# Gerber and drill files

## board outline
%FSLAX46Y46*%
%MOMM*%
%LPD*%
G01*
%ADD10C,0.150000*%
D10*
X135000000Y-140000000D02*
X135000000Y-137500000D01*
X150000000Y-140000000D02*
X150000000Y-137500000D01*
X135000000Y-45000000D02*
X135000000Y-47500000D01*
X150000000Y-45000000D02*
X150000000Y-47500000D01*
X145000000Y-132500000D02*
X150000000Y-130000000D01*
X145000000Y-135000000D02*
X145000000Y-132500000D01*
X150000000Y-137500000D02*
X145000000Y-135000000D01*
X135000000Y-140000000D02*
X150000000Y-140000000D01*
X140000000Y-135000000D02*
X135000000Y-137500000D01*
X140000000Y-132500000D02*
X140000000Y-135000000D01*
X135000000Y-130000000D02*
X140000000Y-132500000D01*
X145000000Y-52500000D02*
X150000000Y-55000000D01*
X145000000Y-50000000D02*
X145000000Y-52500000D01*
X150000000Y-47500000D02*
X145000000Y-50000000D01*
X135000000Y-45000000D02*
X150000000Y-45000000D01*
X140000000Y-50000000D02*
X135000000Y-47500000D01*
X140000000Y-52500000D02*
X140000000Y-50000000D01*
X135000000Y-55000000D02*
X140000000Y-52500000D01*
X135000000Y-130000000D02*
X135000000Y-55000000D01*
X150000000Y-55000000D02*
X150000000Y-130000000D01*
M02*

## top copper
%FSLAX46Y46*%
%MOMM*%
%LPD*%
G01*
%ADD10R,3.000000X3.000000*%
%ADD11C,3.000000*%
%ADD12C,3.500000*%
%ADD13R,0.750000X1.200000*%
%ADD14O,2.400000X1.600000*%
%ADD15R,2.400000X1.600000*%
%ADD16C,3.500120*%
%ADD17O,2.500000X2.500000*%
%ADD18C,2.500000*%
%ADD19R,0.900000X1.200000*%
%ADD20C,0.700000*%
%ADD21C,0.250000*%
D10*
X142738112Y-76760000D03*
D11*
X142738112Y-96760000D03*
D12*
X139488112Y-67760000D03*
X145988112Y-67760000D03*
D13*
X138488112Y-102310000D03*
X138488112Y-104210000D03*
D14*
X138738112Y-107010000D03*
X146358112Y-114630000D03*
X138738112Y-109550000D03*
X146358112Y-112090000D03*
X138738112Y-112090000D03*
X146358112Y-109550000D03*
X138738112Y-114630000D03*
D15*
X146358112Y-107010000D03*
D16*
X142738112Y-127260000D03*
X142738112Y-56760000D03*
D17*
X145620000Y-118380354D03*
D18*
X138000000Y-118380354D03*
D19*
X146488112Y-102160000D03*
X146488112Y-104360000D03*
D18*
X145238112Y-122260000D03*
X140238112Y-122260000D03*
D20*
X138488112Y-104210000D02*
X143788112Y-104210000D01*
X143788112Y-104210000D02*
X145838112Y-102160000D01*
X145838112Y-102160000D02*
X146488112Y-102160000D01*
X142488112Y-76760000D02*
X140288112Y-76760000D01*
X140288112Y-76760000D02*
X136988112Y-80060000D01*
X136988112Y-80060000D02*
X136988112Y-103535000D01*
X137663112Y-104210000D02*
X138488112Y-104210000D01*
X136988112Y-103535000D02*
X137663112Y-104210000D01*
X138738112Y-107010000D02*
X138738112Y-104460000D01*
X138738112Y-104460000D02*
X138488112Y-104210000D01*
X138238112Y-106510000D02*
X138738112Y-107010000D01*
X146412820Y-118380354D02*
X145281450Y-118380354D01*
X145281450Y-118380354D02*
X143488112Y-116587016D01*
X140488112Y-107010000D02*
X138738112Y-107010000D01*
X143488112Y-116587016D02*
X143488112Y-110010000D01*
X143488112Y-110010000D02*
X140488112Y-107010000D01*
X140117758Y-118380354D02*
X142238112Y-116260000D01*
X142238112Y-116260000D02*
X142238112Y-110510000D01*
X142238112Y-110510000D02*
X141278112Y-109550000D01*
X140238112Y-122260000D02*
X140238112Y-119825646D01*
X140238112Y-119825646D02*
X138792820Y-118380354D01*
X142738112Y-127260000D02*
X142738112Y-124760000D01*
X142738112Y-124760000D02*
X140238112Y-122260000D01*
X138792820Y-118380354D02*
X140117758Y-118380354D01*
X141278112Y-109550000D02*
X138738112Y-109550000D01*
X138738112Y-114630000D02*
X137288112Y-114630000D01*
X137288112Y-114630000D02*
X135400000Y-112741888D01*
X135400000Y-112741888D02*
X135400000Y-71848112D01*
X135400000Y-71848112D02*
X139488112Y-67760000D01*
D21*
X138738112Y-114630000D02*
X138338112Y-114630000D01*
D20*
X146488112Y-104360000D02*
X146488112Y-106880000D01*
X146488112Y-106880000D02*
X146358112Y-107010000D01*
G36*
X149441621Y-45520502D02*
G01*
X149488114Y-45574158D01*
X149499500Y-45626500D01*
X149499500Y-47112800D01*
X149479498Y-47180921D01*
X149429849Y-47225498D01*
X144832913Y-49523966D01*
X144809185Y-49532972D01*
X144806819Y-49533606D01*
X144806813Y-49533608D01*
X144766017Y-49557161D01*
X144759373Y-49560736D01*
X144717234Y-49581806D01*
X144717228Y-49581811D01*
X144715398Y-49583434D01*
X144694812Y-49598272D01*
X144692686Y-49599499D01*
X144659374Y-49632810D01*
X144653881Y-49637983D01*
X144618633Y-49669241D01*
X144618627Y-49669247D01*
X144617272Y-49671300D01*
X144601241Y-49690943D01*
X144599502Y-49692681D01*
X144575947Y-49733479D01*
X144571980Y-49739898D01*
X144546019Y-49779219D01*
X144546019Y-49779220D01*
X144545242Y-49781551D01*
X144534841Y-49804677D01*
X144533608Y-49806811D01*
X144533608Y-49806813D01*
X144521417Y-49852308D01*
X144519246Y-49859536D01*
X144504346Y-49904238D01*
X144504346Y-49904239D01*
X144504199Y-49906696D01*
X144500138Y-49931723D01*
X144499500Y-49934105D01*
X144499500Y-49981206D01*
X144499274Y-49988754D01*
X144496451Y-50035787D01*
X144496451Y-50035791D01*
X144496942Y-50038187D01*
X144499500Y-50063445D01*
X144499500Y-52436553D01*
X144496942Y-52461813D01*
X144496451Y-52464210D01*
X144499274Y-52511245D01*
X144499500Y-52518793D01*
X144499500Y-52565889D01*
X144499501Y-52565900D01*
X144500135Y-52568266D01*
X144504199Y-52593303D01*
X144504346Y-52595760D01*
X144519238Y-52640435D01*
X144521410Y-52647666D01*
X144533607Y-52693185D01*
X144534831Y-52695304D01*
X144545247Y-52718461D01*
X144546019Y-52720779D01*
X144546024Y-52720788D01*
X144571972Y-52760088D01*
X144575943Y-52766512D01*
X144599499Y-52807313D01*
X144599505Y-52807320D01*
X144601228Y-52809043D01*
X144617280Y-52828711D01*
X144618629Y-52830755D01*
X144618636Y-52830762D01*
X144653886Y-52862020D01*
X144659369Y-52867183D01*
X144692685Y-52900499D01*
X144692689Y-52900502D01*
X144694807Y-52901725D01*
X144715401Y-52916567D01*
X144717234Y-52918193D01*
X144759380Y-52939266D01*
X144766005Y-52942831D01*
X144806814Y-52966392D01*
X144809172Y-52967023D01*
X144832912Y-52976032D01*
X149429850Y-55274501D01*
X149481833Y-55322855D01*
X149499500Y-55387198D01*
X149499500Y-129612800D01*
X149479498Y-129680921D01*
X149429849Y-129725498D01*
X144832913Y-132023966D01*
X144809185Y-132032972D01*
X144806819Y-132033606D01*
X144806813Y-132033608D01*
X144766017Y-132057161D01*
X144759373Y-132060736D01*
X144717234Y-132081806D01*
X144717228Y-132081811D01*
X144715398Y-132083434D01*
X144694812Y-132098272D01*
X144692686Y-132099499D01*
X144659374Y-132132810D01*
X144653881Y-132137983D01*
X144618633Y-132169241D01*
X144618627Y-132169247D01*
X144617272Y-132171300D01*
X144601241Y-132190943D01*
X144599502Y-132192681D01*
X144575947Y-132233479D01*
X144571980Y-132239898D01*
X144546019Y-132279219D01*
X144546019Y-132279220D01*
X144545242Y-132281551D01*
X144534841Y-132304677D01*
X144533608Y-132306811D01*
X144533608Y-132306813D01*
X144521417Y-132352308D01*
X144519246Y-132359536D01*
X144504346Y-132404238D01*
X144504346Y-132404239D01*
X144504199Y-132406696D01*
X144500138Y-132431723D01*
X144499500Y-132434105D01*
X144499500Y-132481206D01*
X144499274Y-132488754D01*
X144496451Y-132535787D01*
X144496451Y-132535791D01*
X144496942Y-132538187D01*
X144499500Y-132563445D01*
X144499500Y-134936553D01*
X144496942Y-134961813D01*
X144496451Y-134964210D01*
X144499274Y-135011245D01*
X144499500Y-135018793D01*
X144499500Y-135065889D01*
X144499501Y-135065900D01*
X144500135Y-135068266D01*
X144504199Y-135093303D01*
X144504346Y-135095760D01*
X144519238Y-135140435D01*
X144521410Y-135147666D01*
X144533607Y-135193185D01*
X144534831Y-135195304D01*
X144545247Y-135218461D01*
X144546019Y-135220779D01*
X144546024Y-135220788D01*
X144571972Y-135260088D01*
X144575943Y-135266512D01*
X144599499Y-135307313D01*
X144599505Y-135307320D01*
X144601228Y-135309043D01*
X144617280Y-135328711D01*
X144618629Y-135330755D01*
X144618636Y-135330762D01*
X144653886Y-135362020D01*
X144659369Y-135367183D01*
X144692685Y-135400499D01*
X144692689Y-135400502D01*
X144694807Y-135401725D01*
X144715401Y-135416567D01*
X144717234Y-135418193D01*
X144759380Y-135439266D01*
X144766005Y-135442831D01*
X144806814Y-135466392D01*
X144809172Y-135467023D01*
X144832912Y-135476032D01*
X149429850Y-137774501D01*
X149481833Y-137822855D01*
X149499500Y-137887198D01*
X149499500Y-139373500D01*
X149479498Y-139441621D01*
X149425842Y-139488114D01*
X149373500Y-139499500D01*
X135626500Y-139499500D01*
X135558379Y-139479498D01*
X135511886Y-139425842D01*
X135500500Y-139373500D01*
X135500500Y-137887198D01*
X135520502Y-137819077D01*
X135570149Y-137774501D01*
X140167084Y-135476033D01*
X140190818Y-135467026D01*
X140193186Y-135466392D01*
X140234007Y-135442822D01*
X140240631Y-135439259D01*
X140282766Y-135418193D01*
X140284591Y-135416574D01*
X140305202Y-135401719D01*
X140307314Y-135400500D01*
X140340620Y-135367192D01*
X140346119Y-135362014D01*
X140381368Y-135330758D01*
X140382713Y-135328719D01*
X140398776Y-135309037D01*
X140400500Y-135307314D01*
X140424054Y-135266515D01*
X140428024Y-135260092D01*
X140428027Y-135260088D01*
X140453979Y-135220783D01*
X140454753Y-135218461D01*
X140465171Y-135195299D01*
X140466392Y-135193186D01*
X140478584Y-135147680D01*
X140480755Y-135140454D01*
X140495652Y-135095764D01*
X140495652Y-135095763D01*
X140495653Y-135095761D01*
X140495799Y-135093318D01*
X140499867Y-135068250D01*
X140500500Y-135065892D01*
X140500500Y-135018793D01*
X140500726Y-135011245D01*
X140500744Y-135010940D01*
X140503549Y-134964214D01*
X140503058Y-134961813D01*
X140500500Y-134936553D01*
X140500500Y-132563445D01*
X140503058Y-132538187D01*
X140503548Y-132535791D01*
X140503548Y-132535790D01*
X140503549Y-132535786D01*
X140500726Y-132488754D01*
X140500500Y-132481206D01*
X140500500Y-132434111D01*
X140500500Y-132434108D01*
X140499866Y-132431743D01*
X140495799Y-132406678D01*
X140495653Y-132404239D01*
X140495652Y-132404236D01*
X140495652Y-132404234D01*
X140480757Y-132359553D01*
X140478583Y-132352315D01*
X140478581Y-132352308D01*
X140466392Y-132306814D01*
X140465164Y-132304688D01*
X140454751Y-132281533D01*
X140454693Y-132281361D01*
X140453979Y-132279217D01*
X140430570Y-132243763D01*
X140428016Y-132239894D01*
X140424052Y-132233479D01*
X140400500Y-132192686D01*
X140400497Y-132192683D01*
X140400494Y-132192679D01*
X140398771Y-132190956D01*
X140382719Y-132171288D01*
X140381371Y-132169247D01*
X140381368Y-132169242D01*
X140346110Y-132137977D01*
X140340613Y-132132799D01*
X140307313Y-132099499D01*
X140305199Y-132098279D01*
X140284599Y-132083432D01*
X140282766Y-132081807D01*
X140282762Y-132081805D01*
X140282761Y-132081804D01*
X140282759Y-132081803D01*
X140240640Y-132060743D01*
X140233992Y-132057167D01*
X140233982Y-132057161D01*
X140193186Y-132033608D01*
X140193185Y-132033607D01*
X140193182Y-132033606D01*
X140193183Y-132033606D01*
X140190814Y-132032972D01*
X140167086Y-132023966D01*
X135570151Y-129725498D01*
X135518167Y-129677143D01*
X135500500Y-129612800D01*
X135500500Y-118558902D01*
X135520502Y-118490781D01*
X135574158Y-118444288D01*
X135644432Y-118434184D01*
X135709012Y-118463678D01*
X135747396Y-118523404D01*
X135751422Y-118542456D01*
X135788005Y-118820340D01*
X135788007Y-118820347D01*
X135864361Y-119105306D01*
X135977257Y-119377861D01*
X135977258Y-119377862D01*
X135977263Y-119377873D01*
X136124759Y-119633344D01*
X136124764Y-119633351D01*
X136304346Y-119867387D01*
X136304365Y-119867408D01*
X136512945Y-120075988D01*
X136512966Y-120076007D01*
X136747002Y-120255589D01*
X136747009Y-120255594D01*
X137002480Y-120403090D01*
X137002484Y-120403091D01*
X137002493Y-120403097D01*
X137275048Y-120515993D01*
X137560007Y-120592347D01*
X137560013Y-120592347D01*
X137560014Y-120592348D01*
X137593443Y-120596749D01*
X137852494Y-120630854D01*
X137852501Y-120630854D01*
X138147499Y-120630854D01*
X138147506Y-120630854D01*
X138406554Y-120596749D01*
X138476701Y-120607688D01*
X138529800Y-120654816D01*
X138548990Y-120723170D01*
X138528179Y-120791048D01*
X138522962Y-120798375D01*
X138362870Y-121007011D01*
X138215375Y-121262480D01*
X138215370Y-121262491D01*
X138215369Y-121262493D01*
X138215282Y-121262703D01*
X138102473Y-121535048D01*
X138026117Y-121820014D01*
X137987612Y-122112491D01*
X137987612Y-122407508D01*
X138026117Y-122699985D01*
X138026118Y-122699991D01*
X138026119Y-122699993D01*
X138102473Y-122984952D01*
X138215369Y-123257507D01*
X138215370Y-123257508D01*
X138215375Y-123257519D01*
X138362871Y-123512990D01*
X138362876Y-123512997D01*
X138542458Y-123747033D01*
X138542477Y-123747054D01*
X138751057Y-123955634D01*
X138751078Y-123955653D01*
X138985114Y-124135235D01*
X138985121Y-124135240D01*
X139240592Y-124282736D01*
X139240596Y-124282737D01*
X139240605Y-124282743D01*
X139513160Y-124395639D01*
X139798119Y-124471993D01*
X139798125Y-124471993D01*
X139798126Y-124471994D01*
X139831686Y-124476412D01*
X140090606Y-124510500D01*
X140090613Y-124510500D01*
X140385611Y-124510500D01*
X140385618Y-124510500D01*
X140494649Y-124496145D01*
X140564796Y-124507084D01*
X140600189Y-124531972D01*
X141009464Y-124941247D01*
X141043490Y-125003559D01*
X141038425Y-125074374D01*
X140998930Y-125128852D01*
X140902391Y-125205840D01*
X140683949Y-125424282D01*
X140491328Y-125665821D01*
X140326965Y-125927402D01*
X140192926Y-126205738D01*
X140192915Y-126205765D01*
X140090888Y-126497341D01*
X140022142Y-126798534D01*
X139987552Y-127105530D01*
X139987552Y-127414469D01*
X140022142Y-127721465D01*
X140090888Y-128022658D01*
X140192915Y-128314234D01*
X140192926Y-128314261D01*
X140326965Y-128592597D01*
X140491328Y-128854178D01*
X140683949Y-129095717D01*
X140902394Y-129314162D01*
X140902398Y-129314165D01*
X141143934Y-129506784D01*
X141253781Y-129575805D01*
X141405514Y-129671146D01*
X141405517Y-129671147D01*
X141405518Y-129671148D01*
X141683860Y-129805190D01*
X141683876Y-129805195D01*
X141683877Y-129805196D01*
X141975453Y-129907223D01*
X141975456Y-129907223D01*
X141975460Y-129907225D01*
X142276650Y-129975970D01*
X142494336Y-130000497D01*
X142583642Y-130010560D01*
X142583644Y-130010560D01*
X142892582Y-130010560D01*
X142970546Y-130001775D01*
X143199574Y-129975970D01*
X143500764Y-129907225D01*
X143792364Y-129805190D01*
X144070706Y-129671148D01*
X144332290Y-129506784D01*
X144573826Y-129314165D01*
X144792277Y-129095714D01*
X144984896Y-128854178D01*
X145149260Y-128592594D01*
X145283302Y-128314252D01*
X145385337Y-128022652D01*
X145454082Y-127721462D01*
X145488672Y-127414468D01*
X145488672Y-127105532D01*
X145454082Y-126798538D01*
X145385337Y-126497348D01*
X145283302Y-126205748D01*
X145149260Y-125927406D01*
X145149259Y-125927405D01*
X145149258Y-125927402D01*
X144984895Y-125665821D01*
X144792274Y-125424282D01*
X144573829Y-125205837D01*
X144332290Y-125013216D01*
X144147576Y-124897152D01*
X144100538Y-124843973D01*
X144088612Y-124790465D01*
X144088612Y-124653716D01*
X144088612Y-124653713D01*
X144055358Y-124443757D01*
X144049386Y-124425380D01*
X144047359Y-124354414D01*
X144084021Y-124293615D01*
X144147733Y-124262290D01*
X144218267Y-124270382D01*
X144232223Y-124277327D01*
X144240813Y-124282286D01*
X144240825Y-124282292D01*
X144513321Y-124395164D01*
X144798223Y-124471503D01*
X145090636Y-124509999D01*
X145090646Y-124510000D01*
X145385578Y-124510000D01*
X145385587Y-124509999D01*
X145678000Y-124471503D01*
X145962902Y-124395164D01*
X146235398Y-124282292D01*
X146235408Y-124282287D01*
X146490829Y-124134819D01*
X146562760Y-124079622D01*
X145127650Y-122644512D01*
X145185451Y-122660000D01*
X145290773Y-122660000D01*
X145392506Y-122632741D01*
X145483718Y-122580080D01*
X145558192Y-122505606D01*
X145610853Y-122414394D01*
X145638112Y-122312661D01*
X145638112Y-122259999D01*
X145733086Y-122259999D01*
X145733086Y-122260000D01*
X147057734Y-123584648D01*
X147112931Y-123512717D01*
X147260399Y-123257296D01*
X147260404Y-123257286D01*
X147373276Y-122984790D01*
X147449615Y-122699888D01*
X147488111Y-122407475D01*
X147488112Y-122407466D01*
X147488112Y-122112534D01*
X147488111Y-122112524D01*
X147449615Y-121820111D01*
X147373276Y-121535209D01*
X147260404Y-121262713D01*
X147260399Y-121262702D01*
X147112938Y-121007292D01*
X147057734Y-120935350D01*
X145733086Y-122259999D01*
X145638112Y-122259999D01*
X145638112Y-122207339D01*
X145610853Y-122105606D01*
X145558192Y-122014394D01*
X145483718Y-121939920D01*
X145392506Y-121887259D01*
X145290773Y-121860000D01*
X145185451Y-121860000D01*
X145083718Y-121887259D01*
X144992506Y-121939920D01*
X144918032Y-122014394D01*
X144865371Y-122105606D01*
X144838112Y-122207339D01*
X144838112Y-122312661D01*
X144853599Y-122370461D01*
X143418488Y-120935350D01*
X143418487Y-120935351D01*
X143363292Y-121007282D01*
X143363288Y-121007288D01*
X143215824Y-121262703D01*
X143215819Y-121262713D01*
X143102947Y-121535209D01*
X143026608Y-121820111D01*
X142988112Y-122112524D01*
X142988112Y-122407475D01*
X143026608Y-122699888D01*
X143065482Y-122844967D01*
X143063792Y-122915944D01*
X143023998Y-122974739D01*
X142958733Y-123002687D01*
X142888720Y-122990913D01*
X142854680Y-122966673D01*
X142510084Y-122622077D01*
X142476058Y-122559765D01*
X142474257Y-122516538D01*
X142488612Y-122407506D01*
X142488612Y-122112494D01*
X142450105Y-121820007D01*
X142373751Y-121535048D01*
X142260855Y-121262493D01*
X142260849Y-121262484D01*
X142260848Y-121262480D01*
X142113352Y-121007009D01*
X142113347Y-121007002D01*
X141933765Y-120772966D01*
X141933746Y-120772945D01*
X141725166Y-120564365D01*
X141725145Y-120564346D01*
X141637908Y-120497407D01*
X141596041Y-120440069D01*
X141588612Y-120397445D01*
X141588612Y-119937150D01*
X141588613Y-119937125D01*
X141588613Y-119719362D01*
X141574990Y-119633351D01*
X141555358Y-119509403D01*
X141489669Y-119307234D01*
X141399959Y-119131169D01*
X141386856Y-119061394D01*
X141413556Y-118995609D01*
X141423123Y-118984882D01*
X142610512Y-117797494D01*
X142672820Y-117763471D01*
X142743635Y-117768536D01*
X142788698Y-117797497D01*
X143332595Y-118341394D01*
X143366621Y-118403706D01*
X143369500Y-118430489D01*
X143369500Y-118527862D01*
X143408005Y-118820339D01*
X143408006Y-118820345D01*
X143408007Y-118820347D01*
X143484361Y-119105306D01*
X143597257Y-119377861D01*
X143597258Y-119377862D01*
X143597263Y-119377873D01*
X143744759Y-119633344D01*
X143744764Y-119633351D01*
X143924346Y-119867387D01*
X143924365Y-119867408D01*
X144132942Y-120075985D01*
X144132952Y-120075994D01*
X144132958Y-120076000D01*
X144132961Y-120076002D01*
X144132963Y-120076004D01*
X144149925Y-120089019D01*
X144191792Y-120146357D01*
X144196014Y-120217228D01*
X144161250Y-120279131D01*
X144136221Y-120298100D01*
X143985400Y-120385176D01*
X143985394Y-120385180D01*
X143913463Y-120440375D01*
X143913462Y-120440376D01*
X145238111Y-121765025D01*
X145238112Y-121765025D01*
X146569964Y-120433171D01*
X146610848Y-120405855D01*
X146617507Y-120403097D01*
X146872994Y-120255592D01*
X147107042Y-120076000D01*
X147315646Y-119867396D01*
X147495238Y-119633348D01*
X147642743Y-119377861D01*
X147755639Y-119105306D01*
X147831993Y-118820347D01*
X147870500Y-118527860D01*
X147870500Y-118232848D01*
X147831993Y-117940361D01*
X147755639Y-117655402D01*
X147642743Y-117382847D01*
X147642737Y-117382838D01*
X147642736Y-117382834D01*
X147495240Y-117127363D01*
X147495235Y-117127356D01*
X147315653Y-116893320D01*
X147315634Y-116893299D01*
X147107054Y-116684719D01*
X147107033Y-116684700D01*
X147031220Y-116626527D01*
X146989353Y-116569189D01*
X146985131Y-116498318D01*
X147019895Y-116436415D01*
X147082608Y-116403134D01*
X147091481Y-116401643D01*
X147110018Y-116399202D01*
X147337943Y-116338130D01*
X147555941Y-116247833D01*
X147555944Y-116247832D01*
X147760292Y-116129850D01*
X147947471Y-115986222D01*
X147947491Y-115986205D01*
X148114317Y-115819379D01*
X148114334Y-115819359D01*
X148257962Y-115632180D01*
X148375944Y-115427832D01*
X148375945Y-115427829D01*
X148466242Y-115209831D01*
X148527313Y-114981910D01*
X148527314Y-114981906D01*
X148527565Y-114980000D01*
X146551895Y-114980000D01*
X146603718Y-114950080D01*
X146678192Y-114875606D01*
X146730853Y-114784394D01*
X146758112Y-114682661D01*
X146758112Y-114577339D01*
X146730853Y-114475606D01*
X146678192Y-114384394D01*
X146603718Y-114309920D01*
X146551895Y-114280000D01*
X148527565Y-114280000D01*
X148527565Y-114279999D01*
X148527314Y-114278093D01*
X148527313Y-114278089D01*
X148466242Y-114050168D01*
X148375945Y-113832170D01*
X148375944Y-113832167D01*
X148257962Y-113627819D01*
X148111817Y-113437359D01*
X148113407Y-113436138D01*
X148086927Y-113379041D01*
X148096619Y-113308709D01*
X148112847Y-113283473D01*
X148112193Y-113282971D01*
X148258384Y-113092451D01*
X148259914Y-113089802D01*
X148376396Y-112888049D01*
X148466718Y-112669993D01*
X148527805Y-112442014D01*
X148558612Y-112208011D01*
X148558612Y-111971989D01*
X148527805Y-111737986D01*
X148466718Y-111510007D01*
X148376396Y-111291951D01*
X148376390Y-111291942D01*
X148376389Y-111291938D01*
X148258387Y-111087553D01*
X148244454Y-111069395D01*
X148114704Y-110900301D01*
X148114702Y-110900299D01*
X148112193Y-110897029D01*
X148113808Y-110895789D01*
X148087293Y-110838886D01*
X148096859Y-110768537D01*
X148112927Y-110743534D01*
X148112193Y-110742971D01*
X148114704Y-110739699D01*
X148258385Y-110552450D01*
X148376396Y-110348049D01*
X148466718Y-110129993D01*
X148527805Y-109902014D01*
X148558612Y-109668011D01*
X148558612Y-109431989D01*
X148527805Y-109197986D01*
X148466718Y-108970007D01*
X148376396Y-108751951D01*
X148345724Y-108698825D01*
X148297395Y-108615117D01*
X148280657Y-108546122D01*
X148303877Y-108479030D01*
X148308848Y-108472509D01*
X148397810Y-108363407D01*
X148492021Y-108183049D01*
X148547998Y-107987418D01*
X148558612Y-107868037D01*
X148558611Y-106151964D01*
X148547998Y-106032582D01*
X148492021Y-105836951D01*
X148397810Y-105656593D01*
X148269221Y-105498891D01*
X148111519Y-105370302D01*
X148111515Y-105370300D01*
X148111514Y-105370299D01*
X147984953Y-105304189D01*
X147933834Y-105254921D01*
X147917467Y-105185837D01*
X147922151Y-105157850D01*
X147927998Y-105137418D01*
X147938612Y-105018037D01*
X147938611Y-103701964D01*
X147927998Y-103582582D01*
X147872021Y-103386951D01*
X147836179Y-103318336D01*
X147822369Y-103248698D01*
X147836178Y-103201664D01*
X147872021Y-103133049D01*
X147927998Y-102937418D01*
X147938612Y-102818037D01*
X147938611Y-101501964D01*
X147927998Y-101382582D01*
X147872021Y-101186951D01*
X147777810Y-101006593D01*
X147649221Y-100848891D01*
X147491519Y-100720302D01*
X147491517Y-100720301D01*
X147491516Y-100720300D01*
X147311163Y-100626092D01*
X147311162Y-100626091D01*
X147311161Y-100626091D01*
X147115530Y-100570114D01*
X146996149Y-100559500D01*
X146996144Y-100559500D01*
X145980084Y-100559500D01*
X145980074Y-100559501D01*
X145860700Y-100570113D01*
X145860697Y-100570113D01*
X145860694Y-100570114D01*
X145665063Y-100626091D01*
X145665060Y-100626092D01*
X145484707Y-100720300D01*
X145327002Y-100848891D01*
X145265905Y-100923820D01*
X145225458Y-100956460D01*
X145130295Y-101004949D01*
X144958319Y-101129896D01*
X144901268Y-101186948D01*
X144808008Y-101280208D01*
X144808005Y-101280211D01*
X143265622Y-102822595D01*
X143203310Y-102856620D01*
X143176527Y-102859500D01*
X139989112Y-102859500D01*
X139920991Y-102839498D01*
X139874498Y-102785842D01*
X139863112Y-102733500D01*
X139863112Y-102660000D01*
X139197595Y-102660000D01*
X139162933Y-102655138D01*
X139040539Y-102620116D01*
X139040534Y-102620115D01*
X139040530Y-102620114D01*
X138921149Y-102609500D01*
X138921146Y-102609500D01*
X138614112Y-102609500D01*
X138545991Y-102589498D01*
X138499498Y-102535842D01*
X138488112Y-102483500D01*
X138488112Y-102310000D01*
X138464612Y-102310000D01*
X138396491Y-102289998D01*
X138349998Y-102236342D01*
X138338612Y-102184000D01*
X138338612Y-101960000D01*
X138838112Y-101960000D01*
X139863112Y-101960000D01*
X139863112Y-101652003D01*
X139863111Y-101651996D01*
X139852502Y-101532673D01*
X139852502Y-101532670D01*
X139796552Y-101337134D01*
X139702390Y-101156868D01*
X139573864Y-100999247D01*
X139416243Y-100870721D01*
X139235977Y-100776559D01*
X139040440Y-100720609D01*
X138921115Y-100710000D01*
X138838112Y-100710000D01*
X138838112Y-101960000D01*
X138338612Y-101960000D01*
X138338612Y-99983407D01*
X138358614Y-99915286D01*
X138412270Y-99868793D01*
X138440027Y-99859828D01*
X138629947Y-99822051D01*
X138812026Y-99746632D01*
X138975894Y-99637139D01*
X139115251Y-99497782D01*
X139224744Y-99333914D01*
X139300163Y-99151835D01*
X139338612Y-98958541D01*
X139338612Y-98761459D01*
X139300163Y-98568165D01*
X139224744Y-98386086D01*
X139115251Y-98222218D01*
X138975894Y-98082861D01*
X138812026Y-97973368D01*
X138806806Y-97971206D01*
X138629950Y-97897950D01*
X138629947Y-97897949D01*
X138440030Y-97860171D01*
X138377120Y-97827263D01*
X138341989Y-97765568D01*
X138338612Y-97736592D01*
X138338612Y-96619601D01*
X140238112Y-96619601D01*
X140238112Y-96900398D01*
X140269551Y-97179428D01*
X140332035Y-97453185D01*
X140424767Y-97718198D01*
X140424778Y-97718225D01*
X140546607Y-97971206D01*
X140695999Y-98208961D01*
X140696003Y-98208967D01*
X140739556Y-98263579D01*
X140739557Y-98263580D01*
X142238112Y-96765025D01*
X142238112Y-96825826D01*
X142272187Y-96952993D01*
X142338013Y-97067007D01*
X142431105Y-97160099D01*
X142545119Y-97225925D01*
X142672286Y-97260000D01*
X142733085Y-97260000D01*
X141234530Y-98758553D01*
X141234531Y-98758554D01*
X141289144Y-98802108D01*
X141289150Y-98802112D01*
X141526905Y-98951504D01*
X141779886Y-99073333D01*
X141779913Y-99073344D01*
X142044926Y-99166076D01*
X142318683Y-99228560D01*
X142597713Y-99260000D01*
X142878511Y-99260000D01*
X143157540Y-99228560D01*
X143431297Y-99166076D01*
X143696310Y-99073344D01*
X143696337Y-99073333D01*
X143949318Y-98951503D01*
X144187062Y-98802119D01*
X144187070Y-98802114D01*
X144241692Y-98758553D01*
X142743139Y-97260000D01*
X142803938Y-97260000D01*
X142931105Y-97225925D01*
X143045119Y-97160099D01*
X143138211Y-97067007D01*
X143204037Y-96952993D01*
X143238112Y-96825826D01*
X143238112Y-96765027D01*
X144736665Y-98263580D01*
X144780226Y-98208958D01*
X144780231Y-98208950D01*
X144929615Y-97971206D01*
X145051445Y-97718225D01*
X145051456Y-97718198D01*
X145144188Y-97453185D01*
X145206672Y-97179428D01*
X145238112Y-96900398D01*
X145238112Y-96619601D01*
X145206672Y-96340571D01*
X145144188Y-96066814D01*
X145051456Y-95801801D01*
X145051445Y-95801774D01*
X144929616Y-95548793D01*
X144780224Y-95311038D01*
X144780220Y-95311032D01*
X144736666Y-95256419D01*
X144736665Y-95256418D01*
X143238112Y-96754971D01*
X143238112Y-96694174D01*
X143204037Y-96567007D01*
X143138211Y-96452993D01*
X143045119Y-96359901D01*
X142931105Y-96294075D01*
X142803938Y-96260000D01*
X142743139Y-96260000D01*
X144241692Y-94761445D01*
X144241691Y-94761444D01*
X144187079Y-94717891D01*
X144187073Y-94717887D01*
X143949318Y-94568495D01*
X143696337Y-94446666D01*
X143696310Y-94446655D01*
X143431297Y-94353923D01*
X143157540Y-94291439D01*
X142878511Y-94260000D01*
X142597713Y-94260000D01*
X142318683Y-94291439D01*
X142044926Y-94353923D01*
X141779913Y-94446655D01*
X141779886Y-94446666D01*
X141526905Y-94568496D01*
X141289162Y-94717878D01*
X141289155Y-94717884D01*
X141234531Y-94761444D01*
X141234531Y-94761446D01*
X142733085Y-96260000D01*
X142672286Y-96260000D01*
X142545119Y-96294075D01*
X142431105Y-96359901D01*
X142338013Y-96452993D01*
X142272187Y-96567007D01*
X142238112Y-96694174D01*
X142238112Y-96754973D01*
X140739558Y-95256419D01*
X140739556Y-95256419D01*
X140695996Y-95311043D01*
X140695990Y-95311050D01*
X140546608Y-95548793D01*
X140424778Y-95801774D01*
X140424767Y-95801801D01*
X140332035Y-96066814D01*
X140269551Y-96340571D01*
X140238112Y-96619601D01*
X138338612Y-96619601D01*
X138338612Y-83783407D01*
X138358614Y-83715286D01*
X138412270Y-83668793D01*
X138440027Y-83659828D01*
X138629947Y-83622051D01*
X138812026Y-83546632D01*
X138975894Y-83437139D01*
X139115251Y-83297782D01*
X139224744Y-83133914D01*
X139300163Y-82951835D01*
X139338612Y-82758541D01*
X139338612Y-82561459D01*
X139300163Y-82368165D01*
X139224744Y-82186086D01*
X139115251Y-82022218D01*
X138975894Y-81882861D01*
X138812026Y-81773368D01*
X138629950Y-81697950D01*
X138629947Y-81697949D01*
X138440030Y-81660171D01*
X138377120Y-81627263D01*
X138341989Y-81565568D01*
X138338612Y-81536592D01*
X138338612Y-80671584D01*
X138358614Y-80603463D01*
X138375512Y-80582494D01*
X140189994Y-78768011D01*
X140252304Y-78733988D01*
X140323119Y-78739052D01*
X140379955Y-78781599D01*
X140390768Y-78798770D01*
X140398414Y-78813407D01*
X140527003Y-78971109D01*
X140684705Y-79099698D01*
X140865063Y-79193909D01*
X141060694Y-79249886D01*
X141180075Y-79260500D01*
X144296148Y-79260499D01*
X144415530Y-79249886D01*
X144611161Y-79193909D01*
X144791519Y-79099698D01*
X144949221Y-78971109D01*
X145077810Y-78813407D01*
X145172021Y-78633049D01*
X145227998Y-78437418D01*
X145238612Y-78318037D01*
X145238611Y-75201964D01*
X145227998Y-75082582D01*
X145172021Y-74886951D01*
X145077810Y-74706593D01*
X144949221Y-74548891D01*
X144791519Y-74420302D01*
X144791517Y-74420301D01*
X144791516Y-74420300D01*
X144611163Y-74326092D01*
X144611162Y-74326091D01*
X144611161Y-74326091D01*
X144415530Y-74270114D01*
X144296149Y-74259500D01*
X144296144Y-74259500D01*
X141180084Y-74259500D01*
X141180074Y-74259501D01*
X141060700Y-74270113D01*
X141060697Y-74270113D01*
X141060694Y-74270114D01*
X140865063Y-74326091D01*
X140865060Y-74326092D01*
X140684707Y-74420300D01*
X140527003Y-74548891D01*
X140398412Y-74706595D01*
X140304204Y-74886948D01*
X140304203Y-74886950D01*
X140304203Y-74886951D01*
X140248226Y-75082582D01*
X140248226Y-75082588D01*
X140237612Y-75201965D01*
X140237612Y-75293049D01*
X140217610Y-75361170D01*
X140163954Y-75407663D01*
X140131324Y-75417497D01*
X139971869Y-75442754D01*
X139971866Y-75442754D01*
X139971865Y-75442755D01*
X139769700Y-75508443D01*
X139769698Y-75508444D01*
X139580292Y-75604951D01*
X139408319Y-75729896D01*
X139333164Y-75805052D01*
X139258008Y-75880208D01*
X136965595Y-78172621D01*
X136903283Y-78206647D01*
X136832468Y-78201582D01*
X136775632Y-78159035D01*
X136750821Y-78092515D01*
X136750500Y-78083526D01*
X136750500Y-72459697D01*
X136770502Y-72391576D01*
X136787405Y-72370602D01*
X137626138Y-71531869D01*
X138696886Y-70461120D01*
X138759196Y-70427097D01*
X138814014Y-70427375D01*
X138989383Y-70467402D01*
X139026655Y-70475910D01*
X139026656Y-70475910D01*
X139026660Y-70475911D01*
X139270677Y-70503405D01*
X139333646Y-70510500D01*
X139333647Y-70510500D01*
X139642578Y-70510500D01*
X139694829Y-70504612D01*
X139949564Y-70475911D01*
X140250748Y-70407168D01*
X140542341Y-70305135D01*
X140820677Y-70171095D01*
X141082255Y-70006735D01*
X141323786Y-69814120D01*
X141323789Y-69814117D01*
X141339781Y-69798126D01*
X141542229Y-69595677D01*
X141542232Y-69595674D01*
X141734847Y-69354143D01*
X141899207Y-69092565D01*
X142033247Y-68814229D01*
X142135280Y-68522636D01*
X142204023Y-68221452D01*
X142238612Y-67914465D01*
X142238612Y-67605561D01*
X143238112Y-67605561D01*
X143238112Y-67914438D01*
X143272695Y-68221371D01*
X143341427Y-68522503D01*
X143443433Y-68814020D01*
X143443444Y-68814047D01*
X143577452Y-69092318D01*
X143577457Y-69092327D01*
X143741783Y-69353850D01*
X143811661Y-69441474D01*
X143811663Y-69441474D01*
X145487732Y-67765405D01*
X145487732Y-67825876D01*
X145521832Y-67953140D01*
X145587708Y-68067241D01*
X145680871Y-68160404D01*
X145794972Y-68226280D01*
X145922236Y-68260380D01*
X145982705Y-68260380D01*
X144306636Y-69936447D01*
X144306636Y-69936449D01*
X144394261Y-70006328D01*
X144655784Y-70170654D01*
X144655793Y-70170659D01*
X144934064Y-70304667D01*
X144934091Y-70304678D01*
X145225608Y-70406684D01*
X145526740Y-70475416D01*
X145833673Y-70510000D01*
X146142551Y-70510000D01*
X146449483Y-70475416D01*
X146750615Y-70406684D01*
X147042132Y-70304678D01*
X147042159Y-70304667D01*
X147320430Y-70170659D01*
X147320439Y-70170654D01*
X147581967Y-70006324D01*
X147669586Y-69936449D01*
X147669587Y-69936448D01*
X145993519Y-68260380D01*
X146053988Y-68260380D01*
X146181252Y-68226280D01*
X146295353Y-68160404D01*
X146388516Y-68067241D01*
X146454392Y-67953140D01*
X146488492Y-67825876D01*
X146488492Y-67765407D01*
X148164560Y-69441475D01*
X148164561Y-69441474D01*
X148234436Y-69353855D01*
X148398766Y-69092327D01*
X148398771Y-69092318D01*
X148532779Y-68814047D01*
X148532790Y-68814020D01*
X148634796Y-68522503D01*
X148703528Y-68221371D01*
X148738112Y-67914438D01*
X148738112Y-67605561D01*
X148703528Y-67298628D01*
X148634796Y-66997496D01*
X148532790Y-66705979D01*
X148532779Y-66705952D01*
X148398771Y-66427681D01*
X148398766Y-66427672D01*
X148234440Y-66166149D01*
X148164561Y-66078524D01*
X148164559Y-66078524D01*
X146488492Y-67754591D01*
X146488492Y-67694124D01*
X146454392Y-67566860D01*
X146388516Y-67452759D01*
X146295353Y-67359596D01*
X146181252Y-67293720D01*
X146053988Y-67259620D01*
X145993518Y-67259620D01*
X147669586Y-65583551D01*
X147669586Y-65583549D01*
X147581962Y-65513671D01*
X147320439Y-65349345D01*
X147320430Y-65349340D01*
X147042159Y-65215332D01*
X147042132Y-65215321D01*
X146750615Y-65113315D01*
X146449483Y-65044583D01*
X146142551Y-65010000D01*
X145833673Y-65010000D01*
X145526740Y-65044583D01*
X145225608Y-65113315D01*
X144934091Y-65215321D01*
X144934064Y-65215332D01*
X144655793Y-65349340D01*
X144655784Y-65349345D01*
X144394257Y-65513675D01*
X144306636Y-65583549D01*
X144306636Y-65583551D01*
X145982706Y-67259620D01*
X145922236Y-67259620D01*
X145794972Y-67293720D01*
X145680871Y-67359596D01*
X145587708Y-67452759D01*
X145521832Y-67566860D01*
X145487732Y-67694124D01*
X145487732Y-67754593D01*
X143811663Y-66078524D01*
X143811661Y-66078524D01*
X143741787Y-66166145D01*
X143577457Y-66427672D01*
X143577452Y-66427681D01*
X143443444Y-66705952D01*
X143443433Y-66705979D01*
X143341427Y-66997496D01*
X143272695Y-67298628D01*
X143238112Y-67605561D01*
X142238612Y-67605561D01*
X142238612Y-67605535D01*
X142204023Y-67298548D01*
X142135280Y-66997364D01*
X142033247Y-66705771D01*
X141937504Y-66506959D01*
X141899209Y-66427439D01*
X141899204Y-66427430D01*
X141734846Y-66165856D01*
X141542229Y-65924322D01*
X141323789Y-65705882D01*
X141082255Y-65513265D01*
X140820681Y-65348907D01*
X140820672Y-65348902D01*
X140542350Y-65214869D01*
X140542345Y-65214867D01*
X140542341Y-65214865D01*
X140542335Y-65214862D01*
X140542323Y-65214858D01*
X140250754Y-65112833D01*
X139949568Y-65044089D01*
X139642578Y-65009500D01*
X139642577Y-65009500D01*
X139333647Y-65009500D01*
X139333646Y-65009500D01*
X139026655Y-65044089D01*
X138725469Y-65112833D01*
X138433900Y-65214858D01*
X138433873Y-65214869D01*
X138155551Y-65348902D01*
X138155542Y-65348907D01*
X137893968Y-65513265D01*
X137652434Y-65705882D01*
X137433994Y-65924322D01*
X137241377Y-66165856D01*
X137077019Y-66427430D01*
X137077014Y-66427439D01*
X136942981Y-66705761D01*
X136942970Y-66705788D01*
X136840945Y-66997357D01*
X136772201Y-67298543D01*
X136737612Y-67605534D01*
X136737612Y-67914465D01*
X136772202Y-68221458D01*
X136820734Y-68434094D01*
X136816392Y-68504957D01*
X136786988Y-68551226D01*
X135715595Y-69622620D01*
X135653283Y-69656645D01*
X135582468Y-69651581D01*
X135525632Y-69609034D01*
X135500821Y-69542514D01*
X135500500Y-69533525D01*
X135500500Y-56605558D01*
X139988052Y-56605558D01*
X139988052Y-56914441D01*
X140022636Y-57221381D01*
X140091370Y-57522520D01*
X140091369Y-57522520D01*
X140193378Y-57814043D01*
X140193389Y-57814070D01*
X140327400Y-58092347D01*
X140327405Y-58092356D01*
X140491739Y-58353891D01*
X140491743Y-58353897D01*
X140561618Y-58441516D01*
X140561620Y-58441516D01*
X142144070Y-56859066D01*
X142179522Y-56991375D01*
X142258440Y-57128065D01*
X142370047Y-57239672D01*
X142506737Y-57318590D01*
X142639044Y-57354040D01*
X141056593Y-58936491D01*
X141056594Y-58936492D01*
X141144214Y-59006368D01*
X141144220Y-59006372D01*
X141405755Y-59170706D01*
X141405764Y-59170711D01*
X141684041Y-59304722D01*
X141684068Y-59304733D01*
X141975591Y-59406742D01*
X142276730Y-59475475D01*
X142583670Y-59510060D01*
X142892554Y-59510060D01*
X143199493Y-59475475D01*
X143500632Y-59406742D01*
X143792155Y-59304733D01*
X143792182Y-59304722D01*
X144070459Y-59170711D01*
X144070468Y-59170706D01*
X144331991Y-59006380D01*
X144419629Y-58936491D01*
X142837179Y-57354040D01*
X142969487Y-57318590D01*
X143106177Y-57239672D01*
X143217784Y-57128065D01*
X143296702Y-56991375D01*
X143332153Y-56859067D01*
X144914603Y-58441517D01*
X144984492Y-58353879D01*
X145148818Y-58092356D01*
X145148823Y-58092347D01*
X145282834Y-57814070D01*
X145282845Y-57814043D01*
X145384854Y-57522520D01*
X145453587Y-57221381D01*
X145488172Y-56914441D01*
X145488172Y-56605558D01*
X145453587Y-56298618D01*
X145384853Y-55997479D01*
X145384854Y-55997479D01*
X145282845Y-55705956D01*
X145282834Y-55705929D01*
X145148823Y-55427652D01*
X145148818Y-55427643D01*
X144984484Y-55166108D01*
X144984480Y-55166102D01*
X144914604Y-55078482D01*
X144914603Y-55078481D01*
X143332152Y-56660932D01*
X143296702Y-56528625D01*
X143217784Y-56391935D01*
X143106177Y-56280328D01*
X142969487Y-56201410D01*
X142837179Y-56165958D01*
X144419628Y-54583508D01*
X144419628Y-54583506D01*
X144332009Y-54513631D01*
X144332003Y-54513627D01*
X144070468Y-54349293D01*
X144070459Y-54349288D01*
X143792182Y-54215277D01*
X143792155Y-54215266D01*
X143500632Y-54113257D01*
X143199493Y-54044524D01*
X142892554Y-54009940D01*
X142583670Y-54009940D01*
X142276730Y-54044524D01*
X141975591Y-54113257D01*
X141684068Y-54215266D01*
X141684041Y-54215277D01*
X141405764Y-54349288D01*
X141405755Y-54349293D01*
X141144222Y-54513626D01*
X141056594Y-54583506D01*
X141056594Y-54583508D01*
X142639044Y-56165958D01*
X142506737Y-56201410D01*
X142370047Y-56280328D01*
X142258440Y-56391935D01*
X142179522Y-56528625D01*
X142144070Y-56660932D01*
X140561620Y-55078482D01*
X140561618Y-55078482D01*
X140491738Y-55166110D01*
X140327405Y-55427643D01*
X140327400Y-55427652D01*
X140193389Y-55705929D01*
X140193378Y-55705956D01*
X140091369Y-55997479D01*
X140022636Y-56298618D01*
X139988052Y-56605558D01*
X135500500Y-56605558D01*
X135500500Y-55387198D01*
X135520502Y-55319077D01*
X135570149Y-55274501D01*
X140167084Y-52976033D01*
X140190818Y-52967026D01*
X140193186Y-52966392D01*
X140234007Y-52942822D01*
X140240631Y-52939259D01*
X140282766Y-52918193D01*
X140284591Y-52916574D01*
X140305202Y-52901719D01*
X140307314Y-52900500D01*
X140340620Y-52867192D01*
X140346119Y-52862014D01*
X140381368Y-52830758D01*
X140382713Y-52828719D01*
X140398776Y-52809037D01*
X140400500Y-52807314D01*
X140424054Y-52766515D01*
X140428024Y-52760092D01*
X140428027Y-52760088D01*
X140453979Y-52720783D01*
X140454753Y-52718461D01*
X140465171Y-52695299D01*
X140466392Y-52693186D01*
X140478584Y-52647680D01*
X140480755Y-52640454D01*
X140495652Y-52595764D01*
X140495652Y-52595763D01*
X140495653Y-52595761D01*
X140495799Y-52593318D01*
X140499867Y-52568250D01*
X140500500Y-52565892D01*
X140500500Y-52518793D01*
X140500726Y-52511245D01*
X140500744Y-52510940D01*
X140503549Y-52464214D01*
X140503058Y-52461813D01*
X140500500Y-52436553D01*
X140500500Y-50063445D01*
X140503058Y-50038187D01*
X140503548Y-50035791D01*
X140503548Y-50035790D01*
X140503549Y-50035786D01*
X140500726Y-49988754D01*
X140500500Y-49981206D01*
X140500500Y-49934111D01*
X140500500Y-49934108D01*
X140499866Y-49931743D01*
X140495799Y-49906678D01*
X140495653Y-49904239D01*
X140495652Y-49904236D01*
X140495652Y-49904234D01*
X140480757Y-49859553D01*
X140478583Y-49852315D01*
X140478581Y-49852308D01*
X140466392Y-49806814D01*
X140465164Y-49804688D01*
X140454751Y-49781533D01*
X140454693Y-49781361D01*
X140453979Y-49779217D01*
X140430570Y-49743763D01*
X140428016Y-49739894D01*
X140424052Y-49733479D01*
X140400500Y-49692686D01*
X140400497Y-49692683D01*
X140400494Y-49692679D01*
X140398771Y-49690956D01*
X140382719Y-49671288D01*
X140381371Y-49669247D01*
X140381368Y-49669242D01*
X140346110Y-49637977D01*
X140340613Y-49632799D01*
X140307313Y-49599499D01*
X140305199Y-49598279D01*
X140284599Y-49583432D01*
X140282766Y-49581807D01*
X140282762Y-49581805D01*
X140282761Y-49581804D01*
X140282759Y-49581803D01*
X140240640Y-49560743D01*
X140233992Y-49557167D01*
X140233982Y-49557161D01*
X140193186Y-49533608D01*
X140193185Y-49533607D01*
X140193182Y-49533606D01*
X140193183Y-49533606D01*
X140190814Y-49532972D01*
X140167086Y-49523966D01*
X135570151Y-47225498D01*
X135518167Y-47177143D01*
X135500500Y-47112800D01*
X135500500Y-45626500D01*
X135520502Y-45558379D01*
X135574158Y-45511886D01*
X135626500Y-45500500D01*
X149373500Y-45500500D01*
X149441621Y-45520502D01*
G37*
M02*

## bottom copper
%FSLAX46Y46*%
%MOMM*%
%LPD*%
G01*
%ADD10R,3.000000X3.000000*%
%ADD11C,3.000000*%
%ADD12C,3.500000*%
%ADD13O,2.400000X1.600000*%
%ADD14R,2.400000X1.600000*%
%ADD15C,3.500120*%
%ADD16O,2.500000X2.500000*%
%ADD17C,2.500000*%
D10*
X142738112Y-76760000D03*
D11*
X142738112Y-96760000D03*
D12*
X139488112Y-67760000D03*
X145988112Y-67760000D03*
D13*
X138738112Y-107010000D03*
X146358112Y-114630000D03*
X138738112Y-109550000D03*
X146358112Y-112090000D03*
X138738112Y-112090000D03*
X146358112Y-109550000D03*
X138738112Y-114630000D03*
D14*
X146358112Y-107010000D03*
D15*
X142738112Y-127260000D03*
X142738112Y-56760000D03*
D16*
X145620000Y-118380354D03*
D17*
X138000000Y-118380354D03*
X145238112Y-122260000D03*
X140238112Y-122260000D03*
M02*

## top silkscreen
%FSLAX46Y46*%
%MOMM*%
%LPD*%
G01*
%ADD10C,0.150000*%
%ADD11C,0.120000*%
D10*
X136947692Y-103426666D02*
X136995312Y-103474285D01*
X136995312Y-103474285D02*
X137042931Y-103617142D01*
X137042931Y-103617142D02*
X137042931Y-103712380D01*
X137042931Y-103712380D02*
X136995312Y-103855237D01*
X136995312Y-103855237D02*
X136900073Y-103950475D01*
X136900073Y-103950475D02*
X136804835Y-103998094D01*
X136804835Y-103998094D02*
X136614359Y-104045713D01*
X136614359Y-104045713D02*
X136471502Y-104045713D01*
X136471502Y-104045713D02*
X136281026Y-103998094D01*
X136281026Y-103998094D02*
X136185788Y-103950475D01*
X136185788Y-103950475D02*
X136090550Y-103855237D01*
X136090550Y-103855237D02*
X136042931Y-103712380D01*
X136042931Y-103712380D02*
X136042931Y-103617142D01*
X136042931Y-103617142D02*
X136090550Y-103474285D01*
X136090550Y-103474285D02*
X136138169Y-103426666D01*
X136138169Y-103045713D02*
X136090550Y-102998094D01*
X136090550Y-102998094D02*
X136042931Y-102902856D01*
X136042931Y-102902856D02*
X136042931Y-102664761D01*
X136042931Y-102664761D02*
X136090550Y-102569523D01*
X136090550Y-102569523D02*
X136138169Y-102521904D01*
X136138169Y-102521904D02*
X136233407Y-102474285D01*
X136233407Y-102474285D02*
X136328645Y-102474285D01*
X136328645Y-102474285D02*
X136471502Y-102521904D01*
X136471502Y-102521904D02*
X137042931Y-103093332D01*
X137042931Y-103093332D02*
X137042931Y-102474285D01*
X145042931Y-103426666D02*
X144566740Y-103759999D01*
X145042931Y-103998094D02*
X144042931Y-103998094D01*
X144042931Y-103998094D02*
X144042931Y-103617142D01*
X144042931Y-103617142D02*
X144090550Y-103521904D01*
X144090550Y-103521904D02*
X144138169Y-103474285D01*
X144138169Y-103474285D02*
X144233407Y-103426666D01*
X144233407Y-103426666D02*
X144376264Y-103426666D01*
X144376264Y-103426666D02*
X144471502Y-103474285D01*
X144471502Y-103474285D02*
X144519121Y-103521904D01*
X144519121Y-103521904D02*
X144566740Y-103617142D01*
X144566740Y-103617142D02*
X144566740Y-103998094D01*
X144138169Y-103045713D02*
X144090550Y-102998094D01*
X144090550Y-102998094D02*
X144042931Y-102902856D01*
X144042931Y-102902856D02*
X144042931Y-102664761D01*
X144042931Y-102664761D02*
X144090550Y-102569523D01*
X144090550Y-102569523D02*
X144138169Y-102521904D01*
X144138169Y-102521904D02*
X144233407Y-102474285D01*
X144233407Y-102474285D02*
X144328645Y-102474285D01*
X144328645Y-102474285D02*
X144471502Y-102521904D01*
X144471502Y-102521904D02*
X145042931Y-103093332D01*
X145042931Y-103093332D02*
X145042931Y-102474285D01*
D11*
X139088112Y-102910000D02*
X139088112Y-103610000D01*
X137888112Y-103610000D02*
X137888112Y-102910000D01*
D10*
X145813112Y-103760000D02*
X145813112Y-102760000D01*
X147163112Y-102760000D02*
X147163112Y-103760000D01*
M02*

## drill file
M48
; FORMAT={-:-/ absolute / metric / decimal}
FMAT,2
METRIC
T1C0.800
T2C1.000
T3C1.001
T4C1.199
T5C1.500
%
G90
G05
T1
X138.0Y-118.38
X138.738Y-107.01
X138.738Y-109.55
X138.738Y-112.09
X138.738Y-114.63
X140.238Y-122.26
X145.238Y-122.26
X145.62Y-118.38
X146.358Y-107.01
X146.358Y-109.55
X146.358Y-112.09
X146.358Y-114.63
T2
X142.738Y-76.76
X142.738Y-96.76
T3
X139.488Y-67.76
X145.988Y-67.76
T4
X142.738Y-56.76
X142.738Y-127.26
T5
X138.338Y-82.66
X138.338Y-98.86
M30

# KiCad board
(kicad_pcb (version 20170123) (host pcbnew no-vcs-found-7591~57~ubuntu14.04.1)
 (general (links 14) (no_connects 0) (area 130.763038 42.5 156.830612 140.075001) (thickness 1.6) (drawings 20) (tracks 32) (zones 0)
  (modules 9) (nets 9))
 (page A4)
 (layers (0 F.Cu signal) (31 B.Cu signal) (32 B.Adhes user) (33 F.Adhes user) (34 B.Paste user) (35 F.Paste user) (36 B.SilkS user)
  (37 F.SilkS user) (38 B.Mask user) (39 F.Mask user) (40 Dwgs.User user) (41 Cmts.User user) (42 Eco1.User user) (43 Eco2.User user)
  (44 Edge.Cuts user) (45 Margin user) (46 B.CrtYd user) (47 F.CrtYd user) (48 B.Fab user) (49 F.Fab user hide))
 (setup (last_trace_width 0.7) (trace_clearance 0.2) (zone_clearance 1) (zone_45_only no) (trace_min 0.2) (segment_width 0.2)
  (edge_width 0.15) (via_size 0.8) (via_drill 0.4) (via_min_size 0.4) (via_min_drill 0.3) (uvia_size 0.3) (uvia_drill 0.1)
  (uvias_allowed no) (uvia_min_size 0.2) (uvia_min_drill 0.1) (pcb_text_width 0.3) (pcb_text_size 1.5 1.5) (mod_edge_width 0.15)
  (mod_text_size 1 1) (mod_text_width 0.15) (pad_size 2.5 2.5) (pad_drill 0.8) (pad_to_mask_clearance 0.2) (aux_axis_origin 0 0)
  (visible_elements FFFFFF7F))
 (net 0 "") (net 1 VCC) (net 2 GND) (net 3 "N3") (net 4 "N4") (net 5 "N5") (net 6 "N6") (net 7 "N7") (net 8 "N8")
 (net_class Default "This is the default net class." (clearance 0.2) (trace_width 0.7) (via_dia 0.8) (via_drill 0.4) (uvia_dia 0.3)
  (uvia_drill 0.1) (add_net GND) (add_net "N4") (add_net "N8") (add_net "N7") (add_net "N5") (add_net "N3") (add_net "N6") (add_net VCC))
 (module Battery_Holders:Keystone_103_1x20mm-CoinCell (layer B.Cu) (at 142.738112 90.76 270)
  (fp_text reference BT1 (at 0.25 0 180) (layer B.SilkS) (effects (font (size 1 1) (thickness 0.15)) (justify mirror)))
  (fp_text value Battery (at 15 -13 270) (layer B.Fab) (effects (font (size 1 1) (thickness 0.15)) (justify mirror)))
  (pad 1 thru_hole rect (at -14 0 270) (size 3 3) (drill 1) (layers *.Cu *.Mask) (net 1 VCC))
  (pad 2 thru_hole circle (at 6 0 270) (size 3 3) (drill 1) (layers *.Cu *.Mask) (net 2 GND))
  (pad "" np_thru_hole circle (at -8.1 4.4 270) (size 1.5 1.5) (drill 1.5) (layers *.Cu *.Mask))
  (pad "" np_thru_hole circle (at 8.1 4.4 270) (size 1.5 1.5) (drill 1.5) (layers *.Cu *.Mask)))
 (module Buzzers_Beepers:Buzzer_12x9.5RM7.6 (layer B.Cu) (at 142.738112 67.76 180)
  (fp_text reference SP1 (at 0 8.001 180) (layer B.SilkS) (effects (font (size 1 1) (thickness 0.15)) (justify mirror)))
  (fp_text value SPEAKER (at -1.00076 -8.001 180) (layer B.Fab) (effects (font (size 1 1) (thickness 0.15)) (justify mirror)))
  (pad 2 thru_hole circle (at 3.25 0 180) (size 3.5 3.5) (drill 1.00076) (layers *.Cu *.Mask) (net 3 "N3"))
  (pad 1 thru_hole circle (at -3.25 0 180) (size 3.5 3.5) (drill 1.00076) (layers *.Cu *.Mask) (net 2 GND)))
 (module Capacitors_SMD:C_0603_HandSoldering (layer F.Cu) (at 138.488112 103.26 90)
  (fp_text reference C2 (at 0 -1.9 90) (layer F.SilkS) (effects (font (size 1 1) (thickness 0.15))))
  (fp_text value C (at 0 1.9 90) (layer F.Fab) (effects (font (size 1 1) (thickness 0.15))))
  (fp_line (start 0.35 0.6) (end -0.35 0.6) (layer F.SilkS) (width 0.12))
  (fp_line (start -0.35 -0.6) (end 0.35 -0.6) (layer F.SilkS) (width 0.12))
  (pad 2 smd rect (at 0.95 0 90) (size 1.2 0.75) (layers F.Cu F.Paste F.Mask) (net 2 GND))
  (pad 1 smd rect (at -0.95 0 90) (size 1.2 0.75) (layers F.Cu F.Paste F.Mask) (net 1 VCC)))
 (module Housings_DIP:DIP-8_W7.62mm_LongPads (layer B.Cu) (at 146.358112 107.01 180)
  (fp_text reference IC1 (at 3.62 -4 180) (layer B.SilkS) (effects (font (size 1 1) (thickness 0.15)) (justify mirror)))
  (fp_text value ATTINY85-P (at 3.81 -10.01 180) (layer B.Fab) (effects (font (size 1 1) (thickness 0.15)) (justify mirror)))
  (pad 8 thru_hole oval (at 7.62 0 180) (size 2.4 1.6) (drill 0.8) (layers *.Cu *.Mask) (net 1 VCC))
  (pad 4 thru_hole oval (at 0 -7.62 180) (size 2.4 1.6) (drill 0.8) (layers *.Cu *.Mask) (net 2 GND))
  (pad 7 thru_hole oval (at 7.62 -2.54 180) (size 2.4 1.6) (drill 0.8) (layers *.Cu *.Mask) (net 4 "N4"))
  (pad 3 thru_hole oval (at 0 -5.08 180) (size 2.4 1.6) (drill 0.8) (layers *.Cu *.Mask) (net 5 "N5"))
  (pad 6 thru_hole oval (at 7.62 -5.08 180) (size 2.4 1.6) (drill 0.8) (layers *.Cu *.Mask) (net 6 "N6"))
  (pad 2 thru_hole oval (at 0 -2.54 180) (size 2.4 1.6) (drill 0.8) (layers *.Cu *.Mask) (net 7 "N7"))
  (pad 5 thru_hole oval (at 7.62 -7.62 180) (size 2.4 1.6) (drill 0.8) (layers *.Cu *.Mask) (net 3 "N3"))
  (pad 1 thru_hole rect (at 0 0 180) (size 2.4 1.6) (drill 0.8) (layers *.Cu *.Mask) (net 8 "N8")))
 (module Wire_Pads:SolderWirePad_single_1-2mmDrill (layer B.Cu) (at 142.738112 127.26 180)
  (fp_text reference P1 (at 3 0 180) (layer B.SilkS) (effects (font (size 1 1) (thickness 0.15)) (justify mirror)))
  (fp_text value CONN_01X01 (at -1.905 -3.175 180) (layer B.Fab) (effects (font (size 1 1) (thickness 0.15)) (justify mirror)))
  (pad 1 thru_hole circle (at 0 0 180) (size 3.50012 3.50012) (drill 1.19888) (layers *.Cu *.Mask) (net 4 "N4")))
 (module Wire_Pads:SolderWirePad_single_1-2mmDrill (layer B.Cu) (at 142.738112 56.76 180)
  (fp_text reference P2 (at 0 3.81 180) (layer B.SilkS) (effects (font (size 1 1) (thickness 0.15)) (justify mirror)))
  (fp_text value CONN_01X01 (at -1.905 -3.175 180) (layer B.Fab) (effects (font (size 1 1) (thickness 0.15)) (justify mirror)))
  (pad 1 thru_hole circle (at 0 0 180) (size 3.50012 3.50012) (drill 1.19888) (layers *.Cu *.Mask) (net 2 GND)))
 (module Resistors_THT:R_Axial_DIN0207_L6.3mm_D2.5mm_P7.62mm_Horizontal (layer B.Cu) (at 138 118.380354)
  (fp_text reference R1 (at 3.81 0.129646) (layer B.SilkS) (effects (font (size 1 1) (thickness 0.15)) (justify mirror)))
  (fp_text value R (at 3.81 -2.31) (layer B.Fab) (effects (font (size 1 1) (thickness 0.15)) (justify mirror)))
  (pad 2 thru_hole oval (at 7.62 0) (size 2.5 2.5) (drill 0.8) (layers *.Cu *.Mask) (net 1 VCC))
  (pad 1 thru_hole circle (at 0 0) (size 2.5 2.5) (drill 0.8) (layers *.Cu *.Mask) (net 4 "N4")))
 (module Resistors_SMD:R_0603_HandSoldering (layer F.Cu) (at 146.488112 103.26 90)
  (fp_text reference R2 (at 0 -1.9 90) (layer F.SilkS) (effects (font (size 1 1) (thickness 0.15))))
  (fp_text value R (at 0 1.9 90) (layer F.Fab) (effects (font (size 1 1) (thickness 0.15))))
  (fp_line (start -0.5 -0.675) (end 0.5 -0.675) (layer F.SilkS) (width 0.15))
  (fp_line (start 0.5 0.675) (end -0.5 0.675) (layer F.SilkS) (width 0.15))
  (pad 2 smd rect (at 1.1 0 90) (size 1.2 0.9) (layers F.Cu F.Paste F.Mask) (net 1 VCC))
  (pad 1 smd rect (at -1.1 0 90) (size 1.2 0.9) (layers F.Cu F.Paste F.Mask) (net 8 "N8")))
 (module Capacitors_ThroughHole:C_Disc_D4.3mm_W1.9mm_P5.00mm (layer B.Cu) (at 140.238112 122.26)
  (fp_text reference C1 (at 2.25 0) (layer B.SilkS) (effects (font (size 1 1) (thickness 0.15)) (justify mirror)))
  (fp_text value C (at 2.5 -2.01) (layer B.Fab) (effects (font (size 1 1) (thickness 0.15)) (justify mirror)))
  (pad 2 thru_hole circle (at 5 0) (size 2.5 2.5) (drill 0.8) (layers *.Cu *.Mask) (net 2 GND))
  (pad 1 thru_hole circle (at 0 0) (size 2.5 2.5) (drill 0.8) (layers *.Cu *.Mask) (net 4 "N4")))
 (gr_line (start 135 140) (end 135 137.5) (layer Edge.Cuts) (width 0.15))
 (gr_line (start 150 140) (end 150 137.5) (layer Edge.Cuts) (width 0.15))
 (gr_line (start 135 45) (end 135 47.5) (layer Edge.Cuts) (width 0.15))
 (gr_line (start 150 45) (end 150 47.5) (layer Edge.Cuts) (width 0.15))
 (gr_line (start 145 132.5) (end 150 130) (layer Edge.Cuts) (width 0.15))
 (gr_line (start 145 135) (end 145 132.5) (layer Edge.Cuts) (width 0.15))
 (gr_line (start 150 137.5) (end 145 135) (layer Edge.Cuts) (width 0.15))
 (gr_line (start 135 140) (end 150 140) (layer Edge.Cuts) (width 0.15))
 (gr_line (start 140 135) (end 135 137.5) (layer Edge.Cuts) (width 0.15))
 (gr_line (start 140 132.5) (end 140 135) (layer Edge.Cuts) (width 0.15))
 (gr_line (start 135 130) (end 140 132.5) (layer Edge.Cuts) (width 0.15))
 (gr_line (start 145 52.5) (end 150 55) (layer Edge.Cuts) (width 0.15))
 (gr_line (start 145 50) (end 145 52.5) (layer Edge.Cuts) (width 0.15))
 (gr_line (start 150 47.5) (end 145 50) (layer Edge.Cuts) (width 0.15))
 (gr_line (start 135 45) (end 150 45) (layer Edge.Cuts) (width 0.15))
 (gr_line (start 140 50) (end 135 47.5) (layer Edge.Cuts) (width 0.15))
 (gr_line (start 140 52.5) (end 140 50) (layer Edge.Cuts) (width 0.15))
 (gr_line (start 135 55) (end 140 52.5) (layer Edge.Cuts) (width 0.15))
 (gr_line (start 135 130) (end 135 55) (layer Edge.Cuts) (width 0.15))
 (gr_line (start 150 55) (end 150 130) (layer Edge.Cuts) (width 0.15))
 (segment (start 138.488112 104.21) (end 143.788112 104.21) (width 0.7) (layer F.Cu) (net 1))
 (segment (start 143.788112 104.21) (end 145.838112 102.16) (width 0.7) (layer F.Cu) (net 1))
 (segment (start 145.838112 102.16) (end 146.488112 102.16) (width 0.7) (layer F.Cu) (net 1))
 (segment (start 142.488112 76.76) (end 140.288112 76.76) (width 0.7) (layer F.Cu) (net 1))
 (segment (start 140.288112 76.76) (end 136.988112 80.06) (width 0.7) (layer F.Cu) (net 1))
 (segment (start 136.988112 80.06) (end 136.988112 103.535) (width 0.7) (layer F.Cu) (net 1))
 (segment (start 137.663112 104.21) (end 138.488112 104.21) (width 0.7) (layer F.Cu) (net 1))
 (segment (start 136.988112 103.535) (end 137.663112 104.21) (width 0.7) (layer F.Cu) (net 1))
 (segment (start 138.738112 107.01) (end 138.738112 104.46) (width 0.7) (layer F.Cu) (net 1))
 (segment (start 138.738112 104.46) (end 138.488112 104.21) (width 0.7) (layer F.Cu) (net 1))
 (segment (start 138.238112 106.51) (end 138.738112 107.01) (width 0.7) (layer F.Cu) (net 1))
 (segment (start 146.41282 118.380354) (end 145.28145 118.380354) (width 0.7) (layer F.Cu) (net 1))
 (segment (start 145.28145 118.380354) (end 143.488112 116.587016) (width 0.7) (layer F.Cu) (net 1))
 (segment (start 140.488112 107.01) (end 138.738112 107.01) (width 0.7) (layer F.Cu) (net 1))
 (segment (start 143.488112 116.587016) (end 143.488112 110.01) (width 0.7) (layer F.Cu) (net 1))
 (segment (start 143.488112 110.01) (end 140.488112 107.01) (width 0.7) (layer F.Cu) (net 1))
 (segment (start 140.117758 118.380354) (end 142.238112 116.26) (width 0.7) (layer F.Cu) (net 4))
 (segment (start 142.238112 116.26) (end 142.238112 110.51) (width 0.7) (layer F.Cu) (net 4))
 (segment (start 142.238112 110.51) (end 141.278112 109.55) (width 0.7) (layer F.Cu) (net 4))
 (segment (start 140.238112 122.26) (end 140.238112 119.825646) (width 0.7) (layer F.Cu) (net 4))
 (segment (start 140.238112 119.825646) (end 138.79282 118.380354) (width 0.7) (layer F.Cu) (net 4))
 (segment (start 142.738112 127.26) (end 142.738112 124.76) (width 0.7) (layer F.Cu) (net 4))
 (segment (start 142.738112 124.76) (end 140.238112 122.26) (width 0.7) (layer F.Cu) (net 4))
 (segment (start 138.79282 118.380354) (end 140.117758 118.380354) (width 0.7) (layer F.Cu) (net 4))
 (segment (start 141.278112 109.55) (end 138.738112 109.55) (width 0.7) (layer F.Cu) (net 4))
 (segment (start 138.738112 114.63) (end 137.288112 114.63) (width 0.7) (layer F.Cu) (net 3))
 (segment (start 137.288112 114.63) (end 135.4 112.741888) (width 0.7) (layer F.Cu) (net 3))
 (segment (start 135.4 112.741888) (end 135.4 71.848112) (width 0.7) (layer F.Cu) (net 3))
 (segment (start 135.4 71.848112) (end 139.488112 67.76) (width 0.7) (layer F.Cu) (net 3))
 (segment (start 138.738112 114.63) (end 138.338112 114.63) (width 0.25) (layer F.Cu) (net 3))
 (segment (start 146.488112 104.36) (end 146.488112 106.88) (width 0.7) (layer F.Cu) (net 8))
 (segment (start 146.488112 106.88) (end 146.358112 107.01) (width 0.7) (layer F.Cu) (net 8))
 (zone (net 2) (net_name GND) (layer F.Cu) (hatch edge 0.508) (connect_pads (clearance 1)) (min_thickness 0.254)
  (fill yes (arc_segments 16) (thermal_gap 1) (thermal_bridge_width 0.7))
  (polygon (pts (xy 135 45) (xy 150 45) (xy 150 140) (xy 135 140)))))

